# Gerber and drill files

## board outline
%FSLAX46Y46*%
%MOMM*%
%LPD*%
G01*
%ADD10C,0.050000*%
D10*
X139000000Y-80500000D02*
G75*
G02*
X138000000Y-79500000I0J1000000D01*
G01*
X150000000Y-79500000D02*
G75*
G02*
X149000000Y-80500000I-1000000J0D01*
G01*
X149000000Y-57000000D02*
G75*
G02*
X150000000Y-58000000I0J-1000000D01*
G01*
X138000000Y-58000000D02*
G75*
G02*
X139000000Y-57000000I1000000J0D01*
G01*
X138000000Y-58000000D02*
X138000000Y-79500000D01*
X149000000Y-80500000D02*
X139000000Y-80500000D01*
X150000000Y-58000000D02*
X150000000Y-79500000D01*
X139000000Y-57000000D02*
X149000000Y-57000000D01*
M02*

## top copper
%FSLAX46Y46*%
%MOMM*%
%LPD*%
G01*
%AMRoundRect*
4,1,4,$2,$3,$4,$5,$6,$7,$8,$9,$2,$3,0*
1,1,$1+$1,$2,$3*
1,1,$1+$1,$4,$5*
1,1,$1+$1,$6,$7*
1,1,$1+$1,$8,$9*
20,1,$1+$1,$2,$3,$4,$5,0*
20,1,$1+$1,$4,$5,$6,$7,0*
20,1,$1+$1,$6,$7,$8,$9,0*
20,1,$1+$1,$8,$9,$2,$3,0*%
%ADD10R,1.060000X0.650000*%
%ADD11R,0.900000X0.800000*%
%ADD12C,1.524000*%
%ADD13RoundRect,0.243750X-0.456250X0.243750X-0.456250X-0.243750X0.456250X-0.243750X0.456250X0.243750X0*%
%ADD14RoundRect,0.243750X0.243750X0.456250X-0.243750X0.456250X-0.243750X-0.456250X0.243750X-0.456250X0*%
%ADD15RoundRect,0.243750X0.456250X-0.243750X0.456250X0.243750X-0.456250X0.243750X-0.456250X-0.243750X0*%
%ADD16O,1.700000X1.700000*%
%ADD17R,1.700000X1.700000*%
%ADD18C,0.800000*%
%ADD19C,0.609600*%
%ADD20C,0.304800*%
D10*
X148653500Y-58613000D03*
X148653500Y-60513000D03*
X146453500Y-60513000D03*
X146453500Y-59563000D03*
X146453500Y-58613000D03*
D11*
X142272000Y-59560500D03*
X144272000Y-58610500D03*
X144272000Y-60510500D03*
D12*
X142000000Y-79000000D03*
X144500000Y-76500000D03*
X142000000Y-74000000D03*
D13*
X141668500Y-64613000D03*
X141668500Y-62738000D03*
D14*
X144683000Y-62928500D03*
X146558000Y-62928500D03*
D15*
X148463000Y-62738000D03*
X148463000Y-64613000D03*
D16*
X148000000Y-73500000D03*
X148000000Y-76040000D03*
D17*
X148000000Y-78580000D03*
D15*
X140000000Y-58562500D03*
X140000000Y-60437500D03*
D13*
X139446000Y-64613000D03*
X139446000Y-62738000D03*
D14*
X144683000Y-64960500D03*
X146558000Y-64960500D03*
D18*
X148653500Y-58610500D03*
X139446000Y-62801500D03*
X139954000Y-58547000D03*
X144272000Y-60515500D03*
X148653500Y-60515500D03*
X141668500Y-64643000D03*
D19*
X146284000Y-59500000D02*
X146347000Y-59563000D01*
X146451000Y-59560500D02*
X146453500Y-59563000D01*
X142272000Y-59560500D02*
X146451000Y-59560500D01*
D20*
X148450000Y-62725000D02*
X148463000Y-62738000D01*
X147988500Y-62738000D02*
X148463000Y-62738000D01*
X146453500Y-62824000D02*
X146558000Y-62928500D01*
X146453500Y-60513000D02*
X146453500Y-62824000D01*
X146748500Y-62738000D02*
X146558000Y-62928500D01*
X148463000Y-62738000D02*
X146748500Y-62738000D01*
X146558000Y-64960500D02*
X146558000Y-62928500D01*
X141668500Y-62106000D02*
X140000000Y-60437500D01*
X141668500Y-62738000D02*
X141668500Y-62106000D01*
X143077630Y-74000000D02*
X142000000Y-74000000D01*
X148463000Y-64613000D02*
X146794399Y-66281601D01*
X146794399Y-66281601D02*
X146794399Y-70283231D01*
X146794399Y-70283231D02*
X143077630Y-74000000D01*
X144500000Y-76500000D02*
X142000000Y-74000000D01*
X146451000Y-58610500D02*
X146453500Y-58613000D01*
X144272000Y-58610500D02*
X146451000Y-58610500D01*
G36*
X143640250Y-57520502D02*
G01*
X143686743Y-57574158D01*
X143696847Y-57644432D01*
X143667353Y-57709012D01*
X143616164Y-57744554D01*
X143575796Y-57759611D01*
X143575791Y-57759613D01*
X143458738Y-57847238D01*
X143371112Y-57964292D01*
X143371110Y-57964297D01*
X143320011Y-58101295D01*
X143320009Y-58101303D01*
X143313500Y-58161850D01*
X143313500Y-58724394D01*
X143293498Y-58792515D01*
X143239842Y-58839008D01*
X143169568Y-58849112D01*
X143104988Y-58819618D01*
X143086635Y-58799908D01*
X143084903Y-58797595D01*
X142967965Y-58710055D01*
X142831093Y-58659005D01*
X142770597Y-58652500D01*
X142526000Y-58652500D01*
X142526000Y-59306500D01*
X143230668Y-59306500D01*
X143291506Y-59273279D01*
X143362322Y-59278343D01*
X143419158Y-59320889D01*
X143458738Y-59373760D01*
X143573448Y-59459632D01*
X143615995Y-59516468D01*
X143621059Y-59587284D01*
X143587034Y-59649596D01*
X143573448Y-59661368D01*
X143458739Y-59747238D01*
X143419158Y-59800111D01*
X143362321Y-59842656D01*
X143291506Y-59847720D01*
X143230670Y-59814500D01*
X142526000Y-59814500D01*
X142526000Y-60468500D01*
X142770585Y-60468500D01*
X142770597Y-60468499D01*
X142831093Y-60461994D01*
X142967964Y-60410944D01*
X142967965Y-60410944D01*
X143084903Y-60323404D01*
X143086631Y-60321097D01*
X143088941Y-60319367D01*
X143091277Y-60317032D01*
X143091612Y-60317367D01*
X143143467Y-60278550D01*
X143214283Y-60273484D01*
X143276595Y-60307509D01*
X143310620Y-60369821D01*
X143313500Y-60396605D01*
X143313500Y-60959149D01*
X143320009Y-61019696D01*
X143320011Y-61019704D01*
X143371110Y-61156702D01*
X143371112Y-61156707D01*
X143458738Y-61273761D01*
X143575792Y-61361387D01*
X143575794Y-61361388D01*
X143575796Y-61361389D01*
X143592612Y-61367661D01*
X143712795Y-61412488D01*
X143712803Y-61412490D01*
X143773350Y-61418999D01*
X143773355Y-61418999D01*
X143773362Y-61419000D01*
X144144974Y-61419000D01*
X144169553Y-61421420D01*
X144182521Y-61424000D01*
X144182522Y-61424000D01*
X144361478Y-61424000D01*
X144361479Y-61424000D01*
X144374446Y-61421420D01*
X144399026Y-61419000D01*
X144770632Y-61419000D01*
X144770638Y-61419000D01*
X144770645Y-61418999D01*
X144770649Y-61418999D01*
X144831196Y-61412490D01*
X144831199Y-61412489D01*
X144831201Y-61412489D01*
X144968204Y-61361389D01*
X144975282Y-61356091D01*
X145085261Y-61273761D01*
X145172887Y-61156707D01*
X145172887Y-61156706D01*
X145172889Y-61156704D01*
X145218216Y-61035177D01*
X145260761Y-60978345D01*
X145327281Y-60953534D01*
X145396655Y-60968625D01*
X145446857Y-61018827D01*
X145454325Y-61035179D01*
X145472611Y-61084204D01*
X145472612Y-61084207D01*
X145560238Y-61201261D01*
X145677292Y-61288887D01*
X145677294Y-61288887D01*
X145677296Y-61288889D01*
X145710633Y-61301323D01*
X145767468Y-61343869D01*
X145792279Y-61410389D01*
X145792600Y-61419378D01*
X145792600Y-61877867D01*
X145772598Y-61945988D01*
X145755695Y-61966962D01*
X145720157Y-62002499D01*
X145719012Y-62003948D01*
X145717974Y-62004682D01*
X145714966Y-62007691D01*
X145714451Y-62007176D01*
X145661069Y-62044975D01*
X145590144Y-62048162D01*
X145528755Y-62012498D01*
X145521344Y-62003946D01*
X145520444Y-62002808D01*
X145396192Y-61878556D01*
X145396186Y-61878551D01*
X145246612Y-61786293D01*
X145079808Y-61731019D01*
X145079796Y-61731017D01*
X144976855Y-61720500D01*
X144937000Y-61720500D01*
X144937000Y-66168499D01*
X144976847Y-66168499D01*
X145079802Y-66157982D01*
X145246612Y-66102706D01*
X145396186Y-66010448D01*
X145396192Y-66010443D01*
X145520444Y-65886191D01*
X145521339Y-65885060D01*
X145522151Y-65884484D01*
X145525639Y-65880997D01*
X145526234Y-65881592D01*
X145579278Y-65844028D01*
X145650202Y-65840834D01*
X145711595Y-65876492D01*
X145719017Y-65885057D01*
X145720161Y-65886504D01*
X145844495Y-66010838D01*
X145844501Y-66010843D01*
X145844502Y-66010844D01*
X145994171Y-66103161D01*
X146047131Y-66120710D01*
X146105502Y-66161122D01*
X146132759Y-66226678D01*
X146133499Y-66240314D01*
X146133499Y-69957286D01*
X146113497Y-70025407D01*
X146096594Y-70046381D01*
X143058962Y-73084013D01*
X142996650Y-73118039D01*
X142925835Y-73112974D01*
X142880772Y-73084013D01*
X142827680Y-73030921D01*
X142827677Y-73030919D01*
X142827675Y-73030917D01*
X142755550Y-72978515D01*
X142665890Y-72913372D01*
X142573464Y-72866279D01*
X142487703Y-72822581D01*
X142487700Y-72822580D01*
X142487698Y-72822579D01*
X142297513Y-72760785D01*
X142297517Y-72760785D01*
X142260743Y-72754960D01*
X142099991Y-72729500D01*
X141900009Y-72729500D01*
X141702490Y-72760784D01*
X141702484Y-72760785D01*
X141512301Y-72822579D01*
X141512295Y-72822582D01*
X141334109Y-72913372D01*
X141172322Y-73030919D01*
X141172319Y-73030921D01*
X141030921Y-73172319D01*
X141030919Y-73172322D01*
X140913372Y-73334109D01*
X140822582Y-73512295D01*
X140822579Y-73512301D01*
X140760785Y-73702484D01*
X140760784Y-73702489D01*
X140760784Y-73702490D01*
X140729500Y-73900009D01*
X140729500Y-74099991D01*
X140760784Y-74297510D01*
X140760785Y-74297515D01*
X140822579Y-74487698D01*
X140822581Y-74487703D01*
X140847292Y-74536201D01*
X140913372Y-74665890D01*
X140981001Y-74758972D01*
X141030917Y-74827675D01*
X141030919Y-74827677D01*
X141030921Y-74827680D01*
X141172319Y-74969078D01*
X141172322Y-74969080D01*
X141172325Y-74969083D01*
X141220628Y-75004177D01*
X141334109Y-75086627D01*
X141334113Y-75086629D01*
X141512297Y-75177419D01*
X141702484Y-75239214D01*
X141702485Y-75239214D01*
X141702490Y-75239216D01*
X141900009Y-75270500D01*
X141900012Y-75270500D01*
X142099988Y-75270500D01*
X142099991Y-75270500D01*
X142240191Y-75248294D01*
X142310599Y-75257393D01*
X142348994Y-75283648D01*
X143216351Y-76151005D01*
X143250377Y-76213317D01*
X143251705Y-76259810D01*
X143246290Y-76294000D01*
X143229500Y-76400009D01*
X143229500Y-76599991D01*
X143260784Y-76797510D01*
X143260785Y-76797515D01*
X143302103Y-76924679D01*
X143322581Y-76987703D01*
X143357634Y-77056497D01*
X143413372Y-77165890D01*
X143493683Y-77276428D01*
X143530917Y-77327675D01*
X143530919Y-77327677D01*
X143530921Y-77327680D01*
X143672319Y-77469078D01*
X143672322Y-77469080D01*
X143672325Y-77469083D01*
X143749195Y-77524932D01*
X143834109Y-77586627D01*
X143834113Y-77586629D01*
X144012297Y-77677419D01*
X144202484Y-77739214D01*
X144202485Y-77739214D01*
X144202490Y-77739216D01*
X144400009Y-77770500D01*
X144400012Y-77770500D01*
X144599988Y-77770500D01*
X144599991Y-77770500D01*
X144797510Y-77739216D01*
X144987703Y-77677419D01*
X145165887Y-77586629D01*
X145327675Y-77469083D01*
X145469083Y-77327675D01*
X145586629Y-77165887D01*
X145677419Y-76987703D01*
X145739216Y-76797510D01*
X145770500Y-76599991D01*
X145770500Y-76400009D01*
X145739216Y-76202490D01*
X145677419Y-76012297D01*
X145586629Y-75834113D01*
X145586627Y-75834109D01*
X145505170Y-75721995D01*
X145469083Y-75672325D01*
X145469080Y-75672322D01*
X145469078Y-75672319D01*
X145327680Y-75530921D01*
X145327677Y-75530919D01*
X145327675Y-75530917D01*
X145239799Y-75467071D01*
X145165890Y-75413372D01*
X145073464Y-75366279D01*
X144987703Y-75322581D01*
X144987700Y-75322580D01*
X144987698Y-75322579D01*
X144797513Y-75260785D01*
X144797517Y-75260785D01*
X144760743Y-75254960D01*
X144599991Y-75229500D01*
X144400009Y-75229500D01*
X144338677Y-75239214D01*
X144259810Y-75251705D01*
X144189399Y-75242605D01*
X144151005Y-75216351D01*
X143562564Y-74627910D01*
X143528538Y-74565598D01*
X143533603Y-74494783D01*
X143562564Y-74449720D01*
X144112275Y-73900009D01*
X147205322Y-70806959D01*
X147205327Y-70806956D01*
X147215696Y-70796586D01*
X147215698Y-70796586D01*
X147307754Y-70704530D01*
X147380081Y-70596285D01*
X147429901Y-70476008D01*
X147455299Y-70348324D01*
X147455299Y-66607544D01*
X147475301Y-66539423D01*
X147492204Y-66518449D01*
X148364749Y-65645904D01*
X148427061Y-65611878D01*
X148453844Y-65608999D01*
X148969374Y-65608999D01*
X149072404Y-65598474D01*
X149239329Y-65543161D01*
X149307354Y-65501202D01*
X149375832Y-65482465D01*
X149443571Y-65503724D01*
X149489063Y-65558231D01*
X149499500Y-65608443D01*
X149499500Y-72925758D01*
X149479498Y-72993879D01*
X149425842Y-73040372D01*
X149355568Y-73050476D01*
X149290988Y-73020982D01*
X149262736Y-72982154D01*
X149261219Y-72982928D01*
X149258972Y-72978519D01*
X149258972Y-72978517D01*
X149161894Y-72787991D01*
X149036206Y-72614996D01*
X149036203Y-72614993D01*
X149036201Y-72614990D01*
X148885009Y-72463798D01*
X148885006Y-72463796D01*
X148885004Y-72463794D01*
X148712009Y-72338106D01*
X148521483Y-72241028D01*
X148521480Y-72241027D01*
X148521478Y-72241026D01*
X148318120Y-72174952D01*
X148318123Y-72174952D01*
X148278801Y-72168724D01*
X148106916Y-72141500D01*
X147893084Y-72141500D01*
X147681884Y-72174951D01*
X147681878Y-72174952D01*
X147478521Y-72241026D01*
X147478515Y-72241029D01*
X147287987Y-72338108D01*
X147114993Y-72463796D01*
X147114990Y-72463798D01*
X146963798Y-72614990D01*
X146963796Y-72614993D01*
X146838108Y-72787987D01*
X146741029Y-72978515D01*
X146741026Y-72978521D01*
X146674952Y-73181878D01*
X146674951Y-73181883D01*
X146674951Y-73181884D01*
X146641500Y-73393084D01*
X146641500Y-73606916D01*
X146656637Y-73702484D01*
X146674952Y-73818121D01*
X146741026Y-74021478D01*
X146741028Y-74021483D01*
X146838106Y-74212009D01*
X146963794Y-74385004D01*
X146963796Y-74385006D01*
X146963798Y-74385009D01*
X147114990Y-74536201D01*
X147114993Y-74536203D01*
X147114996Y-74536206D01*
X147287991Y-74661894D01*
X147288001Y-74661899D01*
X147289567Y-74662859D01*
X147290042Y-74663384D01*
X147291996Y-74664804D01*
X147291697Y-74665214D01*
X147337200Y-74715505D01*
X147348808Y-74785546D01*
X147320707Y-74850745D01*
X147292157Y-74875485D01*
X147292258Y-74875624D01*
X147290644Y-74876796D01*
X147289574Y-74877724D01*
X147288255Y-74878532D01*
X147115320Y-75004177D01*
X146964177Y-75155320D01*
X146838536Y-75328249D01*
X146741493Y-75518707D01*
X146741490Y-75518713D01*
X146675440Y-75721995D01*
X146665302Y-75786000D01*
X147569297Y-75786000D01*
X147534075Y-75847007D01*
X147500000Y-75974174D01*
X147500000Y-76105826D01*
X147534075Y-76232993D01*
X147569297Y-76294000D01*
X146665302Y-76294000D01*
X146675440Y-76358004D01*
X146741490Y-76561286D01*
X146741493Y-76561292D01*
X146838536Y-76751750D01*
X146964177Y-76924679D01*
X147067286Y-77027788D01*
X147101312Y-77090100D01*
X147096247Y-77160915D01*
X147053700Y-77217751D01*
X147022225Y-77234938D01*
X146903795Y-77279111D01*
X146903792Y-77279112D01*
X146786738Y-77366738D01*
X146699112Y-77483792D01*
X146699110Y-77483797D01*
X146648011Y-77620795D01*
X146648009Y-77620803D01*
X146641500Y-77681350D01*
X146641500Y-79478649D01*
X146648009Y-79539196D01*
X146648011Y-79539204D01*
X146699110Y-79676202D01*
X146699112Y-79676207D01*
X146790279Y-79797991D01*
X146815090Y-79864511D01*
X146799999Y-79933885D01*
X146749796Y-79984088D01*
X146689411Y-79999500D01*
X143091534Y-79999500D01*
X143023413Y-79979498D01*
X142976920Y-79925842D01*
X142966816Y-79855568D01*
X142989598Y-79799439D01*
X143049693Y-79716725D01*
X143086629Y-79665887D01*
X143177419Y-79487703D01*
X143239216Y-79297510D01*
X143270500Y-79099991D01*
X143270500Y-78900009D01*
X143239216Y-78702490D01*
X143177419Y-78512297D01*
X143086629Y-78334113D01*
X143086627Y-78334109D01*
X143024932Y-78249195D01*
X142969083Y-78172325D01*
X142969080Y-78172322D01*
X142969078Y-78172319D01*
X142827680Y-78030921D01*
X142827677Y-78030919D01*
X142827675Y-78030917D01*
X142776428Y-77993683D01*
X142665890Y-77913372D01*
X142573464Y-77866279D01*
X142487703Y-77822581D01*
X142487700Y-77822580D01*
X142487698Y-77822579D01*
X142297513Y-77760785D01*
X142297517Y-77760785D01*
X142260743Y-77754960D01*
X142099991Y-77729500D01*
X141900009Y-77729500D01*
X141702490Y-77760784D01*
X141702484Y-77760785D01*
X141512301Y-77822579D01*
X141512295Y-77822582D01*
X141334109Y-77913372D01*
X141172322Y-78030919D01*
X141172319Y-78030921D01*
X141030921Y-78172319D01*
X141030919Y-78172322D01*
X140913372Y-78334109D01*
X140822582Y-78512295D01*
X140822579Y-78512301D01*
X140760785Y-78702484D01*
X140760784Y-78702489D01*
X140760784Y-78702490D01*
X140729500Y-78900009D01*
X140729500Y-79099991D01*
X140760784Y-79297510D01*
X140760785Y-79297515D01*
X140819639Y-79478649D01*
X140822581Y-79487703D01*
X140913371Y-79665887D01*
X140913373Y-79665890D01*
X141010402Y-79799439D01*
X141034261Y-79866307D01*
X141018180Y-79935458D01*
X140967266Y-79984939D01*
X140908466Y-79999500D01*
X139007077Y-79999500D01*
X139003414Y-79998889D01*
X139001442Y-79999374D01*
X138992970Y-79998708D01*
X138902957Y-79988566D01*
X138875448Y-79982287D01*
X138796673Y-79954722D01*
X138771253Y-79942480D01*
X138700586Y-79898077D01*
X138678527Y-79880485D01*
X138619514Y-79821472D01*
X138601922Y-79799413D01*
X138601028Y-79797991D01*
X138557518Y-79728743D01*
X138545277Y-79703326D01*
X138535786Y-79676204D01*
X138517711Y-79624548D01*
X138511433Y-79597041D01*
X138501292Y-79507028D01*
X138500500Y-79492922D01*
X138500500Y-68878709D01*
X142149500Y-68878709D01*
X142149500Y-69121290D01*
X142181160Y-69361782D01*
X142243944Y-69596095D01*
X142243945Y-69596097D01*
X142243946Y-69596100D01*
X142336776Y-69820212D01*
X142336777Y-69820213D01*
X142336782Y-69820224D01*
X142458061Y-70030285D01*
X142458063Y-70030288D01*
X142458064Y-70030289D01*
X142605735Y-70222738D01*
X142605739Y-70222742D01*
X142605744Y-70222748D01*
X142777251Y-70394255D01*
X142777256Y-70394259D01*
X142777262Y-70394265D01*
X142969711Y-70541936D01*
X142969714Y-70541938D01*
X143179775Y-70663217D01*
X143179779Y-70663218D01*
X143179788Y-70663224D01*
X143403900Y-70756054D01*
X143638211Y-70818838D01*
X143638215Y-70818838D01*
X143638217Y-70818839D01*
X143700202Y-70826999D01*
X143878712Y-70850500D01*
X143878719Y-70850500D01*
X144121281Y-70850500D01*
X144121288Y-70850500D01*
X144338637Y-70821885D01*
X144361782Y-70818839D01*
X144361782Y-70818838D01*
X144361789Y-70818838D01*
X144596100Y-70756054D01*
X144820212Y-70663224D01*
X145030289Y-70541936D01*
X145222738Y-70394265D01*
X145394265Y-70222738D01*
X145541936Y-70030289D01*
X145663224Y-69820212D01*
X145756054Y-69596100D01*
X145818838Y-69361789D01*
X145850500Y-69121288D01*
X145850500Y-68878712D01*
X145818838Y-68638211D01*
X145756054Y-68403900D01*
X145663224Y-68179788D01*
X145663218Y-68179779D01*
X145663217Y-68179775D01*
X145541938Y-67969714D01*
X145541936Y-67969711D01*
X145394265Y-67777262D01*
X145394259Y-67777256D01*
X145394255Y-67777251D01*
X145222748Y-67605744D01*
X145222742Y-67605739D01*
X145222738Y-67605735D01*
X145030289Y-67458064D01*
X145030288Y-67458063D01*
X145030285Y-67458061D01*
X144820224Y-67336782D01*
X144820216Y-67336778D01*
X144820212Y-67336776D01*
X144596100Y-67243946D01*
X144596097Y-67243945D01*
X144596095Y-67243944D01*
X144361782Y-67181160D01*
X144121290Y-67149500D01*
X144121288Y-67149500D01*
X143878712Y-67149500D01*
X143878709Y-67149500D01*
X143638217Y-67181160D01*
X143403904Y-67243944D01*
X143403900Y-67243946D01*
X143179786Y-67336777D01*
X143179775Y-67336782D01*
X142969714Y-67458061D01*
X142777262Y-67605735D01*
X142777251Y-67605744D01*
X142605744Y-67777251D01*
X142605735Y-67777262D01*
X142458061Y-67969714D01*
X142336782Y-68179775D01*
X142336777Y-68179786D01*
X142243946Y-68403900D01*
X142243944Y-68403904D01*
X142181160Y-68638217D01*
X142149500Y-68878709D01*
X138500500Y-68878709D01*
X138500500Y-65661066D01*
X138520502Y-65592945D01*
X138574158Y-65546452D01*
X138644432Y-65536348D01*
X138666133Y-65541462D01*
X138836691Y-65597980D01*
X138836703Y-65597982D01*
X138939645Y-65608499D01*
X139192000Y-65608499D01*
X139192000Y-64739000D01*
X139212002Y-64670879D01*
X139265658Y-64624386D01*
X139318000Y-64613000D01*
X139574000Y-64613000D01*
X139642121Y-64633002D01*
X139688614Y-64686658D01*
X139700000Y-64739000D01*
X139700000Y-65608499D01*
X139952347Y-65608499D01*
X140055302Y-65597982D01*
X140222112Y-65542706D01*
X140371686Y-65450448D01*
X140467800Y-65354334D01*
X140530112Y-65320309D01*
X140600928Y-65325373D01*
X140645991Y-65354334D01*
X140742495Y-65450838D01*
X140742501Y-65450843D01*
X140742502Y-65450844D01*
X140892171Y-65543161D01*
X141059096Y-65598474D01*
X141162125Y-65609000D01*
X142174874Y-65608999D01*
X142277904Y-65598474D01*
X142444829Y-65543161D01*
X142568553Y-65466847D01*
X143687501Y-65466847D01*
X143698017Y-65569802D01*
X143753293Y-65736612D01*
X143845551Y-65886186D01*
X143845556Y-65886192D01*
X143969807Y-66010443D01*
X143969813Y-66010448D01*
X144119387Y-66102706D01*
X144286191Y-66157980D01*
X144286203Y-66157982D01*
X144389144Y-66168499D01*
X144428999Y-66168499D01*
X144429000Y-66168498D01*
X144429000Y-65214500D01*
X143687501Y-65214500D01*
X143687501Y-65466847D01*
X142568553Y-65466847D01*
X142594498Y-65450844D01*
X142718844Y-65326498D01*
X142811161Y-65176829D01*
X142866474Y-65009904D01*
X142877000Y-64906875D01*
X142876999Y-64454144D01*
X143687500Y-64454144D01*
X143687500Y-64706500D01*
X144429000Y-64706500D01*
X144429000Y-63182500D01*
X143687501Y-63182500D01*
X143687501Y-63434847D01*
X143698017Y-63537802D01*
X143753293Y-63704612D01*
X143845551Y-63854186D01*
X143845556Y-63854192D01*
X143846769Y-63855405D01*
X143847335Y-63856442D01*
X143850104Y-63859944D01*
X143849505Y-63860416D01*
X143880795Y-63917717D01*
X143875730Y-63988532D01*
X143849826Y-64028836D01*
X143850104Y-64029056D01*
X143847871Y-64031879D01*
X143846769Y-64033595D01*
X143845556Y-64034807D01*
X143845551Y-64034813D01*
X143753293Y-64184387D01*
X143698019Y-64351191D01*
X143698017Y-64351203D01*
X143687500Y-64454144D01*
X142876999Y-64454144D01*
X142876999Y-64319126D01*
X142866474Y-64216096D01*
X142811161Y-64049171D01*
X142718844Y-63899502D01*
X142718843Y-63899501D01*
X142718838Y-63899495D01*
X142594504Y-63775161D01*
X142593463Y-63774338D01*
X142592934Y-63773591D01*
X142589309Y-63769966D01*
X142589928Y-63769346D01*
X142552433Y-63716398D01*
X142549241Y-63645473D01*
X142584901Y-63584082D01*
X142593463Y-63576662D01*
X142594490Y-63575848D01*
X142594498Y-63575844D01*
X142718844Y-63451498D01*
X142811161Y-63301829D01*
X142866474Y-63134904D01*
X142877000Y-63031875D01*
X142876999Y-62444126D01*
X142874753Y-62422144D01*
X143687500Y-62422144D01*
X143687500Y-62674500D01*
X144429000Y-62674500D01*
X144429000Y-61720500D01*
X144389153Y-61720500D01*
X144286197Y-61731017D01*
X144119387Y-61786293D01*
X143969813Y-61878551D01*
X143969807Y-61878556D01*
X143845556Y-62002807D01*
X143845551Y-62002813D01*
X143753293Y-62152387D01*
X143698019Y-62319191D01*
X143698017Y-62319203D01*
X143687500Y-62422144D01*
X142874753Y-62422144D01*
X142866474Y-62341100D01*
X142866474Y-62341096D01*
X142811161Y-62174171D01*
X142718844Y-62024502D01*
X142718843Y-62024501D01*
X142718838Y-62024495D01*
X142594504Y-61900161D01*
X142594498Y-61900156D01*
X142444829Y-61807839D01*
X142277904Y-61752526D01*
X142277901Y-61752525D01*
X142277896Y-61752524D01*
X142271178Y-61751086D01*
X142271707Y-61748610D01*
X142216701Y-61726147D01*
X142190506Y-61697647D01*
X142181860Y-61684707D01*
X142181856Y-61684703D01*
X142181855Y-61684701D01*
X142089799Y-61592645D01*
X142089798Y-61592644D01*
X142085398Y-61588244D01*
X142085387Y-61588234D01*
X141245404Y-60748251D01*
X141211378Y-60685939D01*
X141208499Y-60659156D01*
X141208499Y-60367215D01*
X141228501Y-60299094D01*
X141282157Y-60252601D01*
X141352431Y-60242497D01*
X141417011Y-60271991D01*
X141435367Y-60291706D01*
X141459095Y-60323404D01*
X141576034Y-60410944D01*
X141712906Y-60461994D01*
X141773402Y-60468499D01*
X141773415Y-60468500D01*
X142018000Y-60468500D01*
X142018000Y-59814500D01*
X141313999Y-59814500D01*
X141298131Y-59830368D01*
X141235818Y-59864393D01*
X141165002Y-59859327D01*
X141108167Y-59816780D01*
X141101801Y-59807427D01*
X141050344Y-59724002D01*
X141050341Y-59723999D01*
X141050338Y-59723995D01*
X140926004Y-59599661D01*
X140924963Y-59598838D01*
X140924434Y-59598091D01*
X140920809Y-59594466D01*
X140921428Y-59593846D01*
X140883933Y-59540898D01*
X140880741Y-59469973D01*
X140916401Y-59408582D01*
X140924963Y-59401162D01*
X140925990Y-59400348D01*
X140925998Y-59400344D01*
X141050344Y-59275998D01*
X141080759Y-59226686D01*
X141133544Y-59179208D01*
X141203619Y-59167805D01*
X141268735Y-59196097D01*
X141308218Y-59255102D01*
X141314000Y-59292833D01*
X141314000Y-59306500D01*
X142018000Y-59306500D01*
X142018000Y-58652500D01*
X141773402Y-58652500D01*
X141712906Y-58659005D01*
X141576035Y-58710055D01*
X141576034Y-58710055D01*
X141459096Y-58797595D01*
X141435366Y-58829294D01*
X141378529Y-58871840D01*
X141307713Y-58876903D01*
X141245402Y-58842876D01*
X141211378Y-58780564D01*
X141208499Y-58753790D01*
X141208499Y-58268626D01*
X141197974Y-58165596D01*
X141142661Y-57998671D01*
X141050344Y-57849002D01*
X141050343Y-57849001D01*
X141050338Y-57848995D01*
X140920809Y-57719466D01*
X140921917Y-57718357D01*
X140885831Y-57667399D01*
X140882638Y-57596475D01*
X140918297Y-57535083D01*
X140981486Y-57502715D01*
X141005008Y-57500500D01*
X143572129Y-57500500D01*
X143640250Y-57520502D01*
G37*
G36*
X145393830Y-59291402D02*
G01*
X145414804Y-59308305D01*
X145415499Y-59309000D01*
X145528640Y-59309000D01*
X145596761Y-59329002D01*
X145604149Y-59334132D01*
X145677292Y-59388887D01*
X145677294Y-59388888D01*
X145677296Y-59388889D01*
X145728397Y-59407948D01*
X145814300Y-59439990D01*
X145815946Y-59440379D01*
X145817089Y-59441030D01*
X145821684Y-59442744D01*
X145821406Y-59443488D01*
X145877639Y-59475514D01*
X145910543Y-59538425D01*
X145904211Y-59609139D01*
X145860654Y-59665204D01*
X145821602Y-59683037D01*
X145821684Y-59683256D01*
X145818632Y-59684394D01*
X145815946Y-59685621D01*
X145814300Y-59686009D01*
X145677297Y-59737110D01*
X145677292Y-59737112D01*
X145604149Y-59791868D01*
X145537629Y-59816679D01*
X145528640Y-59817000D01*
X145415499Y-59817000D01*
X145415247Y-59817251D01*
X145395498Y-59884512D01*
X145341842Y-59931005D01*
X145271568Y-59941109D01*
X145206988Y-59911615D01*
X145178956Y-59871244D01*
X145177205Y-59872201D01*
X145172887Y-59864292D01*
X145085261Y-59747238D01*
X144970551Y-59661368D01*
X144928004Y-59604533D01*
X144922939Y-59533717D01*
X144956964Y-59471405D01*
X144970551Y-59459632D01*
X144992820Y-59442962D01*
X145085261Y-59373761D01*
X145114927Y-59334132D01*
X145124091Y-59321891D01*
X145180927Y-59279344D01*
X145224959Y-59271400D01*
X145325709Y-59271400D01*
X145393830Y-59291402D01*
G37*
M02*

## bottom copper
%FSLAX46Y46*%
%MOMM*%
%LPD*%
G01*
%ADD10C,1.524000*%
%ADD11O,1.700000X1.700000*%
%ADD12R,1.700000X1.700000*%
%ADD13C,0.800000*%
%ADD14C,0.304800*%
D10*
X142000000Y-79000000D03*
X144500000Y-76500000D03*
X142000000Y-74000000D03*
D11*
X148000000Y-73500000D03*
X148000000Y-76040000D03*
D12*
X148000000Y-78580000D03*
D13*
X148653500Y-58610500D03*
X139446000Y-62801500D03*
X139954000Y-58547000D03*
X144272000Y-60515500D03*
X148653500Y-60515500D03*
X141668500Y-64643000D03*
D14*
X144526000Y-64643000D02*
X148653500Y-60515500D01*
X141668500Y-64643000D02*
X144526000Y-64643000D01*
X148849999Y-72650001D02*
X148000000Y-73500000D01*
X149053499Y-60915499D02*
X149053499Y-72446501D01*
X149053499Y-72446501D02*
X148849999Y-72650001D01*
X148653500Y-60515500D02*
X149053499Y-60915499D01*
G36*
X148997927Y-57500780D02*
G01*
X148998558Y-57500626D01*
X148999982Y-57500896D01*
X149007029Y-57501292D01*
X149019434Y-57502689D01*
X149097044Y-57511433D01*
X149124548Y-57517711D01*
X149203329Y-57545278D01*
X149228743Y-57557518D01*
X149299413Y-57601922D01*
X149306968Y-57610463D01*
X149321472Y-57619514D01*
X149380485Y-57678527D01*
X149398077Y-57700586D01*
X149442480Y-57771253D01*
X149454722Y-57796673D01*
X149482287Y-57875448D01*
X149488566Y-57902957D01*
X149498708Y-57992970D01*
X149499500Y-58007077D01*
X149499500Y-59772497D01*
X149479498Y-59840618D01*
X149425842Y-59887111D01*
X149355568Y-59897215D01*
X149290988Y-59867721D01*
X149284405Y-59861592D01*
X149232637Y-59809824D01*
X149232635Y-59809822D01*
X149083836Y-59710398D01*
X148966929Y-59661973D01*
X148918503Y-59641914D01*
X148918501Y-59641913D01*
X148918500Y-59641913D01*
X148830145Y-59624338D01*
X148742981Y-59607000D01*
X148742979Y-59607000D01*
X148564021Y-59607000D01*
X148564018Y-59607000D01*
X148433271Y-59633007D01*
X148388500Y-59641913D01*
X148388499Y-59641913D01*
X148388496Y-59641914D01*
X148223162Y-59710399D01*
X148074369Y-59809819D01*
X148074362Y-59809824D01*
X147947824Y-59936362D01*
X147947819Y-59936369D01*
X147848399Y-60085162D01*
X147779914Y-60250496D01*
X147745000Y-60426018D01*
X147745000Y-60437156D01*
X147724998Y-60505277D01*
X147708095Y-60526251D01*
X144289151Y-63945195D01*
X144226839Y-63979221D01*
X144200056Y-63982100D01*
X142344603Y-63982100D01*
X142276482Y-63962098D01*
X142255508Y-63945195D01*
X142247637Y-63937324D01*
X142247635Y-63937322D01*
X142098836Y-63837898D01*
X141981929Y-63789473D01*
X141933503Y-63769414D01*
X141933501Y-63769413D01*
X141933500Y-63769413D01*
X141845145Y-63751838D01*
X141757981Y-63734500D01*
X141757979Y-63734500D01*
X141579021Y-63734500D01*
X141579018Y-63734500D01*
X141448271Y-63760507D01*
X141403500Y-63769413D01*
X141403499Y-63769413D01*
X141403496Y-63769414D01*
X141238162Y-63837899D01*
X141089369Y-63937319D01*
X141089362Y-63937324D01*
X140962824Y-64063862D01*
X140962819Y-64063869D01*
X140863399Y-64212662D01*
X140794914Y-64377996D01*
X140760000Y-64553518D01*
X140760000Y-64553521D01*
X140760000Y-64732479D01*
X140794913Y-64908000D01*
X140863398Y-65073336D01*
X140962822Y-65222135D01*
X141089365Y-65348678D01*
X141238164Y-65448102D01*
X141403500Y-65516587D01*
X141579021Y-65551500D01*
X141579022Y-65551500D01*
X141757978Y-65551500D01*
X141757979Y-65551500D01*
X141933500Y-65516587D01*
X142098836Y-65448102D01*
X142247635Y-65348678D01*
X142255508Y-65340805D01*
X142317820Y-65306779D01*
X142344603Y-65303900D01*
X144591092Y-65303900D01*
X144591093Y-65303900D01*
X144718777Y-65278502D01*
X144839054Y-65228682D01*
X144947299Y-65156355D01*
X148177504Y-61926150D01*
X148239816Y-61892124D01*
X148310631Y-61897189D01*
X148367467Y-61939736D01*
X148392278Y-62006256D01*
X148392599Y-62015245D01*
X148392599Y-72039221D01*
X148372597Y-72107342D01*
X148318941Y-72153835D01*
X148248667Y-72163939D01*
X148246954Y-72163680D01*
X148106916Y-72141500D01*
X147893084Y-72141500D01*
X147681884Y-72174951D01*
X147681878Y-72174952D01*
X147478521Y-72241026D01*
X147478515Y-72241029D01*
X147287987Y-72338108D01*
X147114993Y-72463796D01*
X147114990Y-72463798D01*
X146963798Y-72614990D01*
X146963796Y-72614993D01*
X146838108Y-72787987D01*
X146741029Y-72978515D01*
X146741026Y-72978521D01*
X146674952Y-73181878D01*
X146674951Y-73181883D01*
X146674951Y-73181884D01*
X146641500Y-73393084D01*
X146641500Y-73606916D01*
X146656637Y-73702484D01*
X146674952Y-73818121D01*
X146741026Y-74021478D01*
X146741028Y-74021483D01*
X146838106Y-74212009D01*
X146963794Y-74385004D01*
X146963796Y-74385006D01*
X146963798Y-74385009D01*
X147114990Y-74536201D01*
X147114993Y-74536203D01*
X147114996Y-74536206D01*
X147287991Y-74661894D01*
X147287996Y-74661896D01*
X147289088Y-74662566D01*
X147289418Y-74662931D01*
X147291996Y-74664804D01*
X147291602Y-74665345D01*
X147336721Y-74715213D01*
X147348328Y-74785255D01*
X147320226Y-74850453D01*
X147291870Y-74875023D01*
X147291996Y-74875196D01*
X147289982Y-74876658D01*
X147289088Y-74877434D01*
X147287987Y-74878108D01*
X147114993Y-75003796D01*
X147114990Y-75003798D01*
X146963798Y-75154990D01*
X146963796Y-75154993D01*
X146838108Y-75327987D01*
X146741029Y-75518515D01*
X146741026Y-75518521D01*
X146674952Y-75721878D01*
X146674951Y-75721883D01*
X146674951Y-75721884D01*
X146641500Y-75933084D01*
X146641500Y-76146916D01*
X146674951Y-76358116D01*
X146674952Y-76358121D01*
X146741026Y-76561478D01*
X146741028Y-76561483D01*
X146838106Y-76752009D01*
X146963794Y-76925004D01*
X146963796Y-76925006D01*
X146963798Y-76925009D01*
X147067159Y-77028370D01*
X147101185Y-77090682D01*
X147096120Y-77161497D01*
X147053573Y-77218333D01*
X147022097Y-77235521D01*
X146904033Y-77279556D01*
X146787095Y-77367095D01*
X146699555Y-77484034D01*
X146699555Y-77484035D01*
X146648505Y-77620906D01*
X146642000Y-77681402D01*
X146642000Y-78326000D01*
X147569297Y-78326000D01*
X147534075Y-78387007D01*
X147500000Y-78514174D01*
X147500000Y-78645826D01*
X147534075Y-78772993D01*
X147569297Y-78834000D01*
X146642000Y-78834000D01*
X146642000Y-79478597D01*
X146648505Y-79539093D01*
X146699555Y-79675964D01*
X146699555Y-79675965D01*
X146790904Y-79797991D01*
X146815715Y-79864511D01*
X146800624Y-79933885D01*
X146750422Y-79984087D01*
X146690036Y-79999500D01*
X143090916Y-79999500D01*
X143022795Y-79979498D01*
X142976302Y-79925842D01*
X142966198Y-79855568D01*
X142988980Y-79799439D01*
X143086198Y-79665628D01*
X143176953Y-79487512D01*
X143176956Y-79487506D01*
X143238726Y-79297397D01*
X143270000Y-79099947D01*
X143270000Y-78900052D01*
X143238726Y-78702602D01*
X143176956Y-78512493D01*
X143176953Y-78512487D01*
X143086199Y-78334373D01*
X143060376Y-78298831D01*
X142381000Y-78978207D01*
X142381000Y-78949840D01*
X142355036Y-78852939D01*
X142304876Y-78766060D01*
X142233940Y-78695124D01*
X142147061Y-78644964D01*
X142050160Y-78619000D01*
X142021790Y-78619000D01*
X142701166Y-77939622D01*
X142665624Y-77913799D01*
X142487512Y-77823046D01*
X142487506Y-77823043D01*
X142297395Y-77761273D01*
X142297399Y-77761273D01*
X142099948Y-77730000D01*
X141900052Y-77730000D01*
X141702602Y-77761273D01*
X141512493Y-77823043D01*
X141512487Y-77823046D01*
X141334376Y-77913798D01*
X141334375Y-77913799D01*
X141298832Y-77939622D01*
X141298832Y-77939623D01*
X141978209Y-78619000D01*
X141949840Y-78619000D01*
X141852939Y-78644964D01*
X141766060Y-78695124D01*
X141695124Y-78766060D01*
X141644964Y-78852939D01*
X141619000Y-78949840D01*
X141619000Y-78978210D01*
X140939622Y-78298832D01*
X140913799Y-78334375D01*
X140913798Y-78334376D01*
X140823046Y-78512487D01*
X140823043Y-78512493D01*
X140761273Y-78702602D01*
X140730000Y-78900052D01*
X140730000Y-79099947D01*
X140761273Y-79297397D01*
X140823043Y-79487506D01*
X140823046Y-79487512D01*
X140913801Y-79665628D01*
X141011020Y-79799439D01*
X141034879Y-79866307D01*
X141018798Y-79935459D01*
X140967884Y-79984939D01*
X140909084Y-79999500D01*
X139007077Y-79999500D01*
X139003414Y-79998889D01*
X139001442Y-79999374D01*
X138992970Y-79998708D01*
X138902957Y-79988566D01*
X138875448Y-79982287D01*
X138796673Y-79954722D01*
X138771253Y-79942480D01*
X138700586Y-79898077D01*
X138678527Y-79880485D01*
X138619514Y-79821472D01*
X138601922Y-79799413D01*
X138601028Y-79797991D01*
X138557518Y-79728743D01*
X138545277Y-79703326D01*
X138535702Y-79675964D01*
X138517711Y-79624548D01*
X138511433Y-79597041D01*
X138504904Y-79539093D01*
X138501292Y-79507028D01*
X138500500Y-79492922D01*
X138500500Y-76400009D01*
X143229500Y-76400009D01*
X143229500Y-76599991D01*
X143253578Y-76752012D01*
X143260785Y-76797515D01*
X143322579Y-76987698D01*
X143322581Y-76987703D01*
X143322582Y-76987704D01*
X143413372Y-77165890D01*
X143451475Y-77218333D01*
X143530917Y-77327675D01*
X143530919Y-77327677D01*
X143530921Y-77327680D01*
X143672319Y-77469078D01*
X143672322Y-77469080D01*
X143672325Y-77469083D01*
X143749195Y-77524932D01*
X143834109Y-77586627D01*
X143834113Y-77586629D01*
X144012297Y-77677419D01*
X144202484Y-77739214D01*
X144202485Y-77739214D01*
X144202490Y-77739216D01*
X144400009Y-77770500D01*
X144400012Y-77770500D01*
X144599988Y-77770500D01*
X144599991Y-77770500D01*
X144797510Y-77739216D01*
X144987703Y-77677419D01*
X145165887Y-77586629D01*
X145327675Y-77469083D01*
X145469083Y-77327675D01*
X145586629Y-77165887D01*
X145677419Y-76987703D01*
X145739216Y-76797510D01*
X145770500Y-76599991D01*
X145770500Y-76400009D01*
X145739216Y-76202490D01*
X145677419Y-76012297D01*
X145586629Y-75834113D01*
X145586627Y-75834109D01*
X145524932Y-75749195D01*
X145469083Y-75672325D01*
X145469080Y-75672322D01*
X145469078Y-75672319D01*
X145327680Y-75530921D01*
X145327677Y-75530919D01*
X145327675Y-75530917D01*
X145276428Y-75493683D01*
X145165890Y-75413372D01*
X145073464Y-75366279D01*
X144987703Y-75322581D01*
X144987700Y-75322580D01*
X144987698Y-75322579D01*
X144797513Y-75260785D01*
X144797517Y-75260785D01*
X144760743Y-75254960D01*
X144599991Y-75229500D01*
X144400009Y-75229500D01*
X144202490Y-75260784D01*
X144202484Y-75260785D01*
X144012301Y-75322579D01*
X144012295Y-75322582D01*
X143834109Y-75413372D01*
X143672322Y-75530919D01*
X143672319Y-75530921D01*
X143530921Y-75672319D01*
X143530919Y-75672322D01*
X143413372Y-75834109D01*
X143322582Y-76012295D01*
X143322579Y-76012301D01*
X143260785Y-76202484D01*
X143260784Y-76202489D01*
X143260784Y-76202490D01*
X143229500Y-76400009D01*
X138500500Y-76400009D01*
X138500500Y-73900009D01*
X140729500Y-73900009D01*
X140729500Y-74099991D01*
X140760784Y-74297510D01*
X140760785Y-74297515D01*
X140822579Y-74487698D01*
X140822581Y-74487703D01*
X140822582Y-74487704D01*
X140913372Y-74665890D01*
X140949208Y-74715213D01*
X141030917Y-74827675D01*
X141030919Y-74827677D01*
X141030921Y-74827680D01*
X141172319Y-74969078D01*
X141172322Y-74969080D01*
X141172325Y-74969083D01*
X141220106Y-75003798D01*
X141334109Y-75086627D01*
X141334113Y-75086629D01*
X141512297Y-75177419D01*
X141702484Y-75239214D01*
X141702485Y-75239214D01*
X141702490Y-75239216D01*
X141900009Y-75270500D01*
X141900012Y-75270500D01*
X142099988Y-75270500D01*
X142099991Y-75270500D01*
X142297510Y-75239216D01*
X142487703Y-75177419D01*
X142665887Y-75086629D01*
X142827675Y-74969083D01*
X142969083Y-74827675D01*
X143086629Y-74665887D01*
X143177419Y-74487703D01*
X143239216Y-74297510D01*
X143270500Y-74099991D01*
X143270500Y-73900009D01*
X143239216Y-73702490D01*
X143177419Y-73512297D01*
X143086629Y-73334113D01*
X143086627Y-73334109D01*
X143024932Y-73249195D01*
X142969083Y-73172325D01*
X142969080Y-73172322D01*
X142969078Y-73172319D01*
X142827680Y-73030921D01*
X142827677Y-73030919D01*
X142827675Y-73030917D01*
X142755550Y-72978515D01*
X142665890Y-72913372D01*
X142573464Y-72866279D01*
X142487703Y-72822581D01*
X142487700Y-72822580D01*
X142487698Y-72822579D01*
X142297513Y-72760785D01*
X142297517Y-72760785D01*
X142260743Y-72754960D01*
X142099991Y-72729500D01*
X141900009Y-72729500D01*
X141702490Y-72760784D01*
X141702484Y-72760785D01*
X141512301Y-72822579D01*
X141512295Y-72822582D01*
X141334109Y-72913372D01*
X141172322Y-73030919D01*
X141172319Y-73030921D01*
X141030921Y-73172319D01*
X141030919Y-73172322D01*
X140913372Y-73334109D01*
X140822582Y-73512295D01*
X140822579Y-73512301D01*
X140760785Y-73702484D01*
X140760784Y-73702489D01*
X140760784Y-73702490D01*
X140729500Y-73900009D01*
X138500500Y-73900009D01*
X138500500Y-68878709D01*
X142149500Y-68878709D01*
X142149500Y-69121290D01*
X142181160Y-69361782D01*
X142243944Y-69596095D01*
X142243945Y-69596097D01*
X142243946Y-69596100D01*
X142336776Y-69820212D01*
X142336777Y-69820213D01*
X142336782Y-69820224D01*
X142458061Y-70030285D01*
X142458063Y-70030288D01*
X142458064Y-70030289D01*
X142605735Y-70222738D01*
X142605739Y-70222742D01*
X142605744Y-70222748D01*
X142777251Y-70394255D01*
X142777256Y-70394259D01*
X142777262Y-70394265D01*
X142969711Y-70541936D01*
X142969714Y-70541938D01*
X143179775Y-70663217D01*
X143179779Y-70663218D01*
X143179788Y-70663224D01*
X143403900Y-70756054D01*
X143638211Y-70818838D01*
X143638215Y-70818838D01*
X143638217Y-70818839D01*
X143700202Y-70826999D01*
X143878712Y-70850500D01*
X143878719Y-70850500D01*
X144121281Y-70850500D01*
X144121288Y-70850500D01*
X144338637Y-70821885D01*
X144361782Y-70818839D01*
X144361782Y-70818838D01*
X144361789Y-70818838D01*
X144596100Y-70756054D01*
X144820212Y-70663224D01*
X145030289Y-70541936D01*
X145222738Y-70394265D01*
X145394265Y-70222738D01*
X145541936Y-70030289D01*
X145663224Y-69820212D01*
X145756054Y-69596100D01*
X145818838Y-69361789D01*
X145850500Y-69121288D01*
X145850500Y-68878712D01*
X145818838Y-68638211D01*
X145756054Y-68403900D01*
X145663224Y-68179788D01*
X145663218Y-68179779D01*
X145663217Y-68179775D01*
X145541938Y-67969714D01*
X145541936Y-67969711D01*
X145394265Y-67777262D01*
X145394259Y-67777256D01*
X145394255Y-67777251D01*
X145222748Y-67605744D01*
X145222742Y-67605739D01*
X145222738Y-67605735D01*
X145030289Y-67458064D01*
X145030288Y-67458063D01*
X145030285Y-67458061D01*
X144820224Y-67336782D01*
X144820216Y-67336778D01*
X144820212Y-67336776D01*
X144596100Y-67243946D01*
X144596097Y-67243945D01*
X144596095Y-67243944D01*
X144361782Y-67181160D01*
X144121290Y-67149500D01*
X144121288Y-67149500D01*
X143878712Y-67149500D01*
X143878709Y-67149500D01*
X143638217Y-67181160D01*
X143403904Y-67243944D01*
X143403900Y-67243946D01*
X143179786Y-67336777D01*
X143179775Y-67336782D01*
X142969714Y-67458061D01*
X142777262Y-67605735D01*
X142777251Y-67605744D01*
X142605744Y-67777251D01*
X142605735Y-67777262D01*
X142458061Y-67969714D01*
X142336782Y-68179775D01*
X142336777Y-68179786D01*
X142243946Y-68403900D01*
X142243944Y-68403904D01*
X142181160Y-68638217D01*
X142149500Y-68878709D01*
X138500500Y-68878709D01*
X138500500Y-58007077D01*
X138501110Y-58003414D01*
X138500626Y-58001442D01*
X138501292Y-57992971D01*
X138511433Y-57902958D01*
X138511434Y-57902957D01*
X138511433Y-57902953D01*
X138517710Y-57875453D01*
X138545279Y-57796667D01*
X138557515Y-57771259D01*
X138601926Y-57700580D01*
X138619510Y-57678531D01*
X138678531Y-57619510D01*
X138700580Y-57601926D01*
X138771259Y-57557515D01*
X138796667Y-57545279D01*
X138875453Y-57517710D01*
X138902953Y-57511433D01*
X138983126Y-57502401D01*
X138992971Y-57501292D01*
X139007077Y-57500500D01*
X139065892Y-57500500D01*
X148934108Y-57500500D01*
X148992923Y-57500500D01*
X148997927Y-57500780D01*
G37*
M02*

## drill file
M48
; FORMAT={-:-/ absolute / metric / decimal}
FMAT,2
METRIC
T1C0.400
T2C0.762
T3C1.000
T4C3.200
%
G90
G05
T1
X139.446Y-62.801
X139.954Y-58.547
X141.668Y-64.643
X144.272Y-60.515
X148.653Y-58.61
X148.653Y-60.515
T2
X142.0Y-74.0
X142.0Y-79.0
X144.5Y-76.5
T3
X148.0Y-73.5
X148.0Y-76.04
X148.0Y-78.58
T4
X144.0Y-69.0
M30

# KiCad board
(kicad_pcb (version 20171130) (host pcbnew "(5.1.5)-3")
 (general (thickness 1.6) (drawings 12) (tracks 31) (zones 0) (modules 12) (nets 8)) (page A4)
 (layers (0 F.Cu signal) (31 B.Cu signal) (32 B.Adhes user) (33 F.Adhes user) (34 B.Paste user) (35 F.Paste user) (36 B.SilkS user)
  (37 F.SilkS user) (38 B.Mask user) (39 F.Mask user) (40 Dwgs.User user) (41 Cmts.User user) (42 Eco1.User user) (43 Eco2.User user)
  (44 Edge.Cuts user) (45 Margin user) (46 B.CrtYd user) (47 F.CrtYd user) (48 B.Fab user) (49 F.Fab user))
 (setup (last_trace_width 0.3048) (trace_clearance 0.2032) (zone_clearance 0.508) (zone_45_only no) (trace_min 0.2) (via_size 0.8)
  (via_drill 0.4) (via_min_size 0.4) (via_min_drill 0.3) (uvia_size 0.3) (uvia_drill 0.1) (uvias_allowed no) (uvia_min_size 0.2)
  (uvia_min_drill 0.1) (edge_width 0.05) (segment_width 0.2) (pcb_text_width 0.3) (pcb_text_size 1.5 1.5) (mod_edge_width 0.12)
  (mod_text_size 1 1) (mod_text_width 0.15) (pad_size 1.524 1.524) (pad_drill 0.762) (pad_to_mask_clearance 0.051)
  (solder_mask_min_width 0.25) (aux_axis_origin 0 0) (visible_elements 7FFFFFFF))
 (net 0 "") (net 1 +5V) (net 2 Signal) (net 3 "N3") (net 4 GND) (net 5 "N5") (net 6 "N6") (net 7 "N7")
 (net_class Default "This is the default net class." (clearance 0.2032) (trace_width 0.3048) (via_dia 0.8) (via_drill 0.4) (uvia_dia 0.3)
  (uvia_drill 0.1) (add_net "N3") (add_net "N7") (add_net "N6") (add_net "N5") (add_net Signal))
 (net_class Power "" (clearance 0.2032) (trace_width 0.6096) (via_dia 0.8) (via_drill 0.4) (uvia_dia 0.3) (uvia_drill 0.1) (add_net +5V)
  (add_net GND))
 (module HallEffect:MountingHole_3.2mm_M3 (layer F.Cu) (at 144 69)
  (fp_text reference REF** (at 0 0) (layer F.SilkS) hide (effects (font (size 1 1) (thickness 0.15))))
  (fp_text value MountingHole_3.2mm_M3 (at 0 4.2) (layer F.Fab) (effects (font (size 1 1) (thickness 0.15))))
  (pad 1 np_thru_hole circle (at 0 0) (size 3.2 3.2) (drill 3.2) (layers *.Cu *.Mask)))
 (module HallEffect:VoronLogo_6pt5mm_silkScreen (layer B.Cu) (at 144 61 270)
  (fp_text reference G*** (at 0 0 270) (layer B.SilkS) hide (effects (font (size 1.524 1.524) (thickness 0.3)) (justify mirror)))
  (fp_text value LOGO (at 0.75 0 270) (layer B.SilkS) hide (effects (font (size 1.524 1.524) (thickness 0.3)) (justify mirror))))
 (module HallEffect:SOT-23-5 (layer F.Cu) (at 147.5535 59.563)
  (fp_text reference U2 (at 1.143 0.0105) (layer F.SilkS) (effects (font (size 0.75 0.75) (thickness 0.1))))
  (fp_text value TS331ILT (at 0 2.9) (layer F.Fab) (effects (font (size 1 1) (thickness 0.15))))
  (pad 5 smd rect (at 1.1 -0.95) (size 1.06 0.65) (layers F.Cu F.Paste F.Mask) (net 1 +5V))
  (pad 4 smd rect (at 1.1 0.95) (size 1.06 0.65) (layers F.Cu F.Paste F.Mask) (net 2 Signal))
  (pad 3 smd rect (at -1.1 0.95) (size 1.06 0.65) (layers F.Cu F.Paste F.Mask) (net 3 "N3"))
  (pad 2 smd rect (at -1.1 0) (size 1.06 0.65) (layers F.Cu F.Paste F.Mask) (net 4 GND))
  (pad 1 smd rect (at -1.1 -0.95) (size 1.06 0.65) (layers F.Cu F.Paste F.Mask) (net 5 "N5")))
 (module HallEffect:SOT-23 (layer F.Cu) (at 143.272 59.5605 180)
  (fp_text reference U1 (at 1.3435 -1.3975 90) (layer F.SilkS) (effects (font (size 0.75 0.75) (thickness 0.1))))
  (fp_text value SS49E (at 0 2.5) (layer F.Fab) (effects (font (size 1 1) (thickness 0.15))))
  (pad 3 smd rect (at 1 0 180) (size 0.9 0.8) (layers F.Cu F.Paste F.Mask) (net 4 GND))
  (pad 2 smd rect (at -1 0.95 180) (size 0.9 0.8) (layers F.Cu F.Paste F.Mask) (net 5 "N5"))
  (pad 1 smd rect (at -1 -0.95 180) (size 0.9 0.8) (layers F.Cu F.Paste F.Mask) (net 1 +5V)))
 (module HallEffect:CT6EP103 (layer F.Cu) (at 142 76.5 270)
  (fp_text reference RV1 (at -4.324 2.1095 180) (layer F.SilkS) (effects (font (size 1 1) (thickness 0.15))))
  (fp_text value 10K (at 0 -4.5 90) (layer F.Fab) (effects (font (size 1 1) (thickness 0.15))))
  (pad 3 thru_hole circle (at 2.5 0 270) (size 1.524 1.524) (drill 0.762) (layers *.Cu *.Mask) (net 1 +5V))
  (pad 2 thru_hole circle (at 0 -2.5 270) (size 1.524 1.524) (drill 0.762) (layers *.Cu *.Mask) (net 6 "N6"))
  (pad 1 thru_hole circle (at -2.5 0 270) (size 1.524 1.524) (drill 0.762) (layers *.Cu *.Mask) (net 6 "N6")))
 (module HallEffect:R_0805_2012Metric (layer F.Cu) (at 141.6685 63.6755 270)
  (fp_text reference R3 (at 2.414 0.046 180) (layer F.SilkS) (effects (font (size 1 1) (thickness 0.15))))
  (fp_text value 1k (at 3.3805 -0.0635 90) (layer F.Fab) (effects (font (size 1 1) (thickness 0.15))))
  (pad 2 smd roundrect (at 0.9375 0 270) (size 0.975 1.4) (layers F.Cu F.Paste F.Mask) (roundrect_rratio 0.25) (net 2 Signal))
  (pad 1 smd roundrect (at -0.9375 0 270) (size 0.975 1.4) (layers F.Cu F.Paste F.Mask) (roundrect_rratio 0.25) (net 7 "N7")))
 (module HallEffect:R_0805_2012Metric (layer F.Cu) (at 145.6205 62.9285 180)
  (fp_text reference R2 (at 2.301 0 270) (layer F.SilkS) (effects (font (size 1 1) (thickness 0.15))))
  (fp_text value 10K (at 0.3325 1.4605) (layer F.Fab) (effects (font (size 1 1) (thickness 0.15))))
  (pad 2 smd roundrect (at 0.9375 0 180) (size 0.975 1.4) (layers F.Cu F.Paste F.Mask) (roundrect_rratio 0.25) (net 4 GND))
  (pad 1 smd roundrect (at -0.9375 0 180) (size 0.975 1.4) (layers F.Cu F.Paste F.Mask) (roundrect_rratio 0.25) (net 3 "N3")))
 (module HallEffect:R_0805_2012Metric (layer F.Cu) (at 148.463 63.6755 90)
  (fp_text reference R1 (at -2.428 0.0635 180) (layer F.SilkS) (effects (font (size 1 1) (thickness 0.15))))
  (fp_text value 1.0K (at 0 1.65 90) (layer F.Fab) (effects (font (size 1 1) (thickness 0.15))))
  (pad 2 smd roundrect (at 0.9375 0 90) (size 0.975 1.4) (layers F.Cu F.Paste F.Mask) (roundrect_rratio 0.25) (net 3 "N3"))
  (pad 1 smd roundrect (at -0.9375 0 90) (size 0.975 1.4) (layers F.Cu F.Paste F.Mask) (roundrect_rratio 0.25) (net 6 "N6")))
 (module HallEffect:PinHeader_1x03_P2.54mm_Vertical (layer F.Cu) (at 148 78.58 180)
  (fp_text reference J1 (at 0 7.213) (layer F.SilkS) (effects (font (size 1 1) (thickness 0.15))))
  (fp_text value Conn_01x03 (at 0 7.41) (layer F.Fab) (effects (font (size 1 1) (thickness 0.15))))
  (pad 3 thru_hole oval (at 0 5.08 180) (size 1.7 1.7) (drill 1) (layers *.Cu *.Mask) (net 2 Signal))
  (pad 2 thru_hole oval (at 0 2.54 180) (size 1.7 1.7) (drill 1) (layers *.Cu *.Mask) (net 4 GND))
  (pad 1 thru_hole rect (at 0 0 180) (size 1.7 1.7) (drill 1) (layers *.Cu *.Mask) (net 1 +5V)))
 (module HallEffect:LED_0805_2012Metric (layer F.Cu) (at 140 59.5 90)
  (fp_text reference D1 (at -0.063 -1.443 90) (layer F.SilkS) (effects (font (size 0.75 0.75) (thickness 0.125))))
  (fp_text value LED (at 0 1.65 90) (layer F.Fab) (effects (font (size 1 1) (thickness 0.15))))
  (pad 2 smd roundrect (at 0.9375 0 90) (size 0.975 1.4) (layers F.Cu F.Paste F.Mask) (roundrect_rratio 0.25) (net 1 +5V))
  (pad 1 smd roundrect (at -0.9375 0 90) (size 0.975 1.4) (layers F.Cu F.Paste F.Mask) (roundrect_rratio 0.25) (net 7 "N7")))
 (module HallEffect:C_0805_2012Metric (layer F.Cu) (at 139.446 63.6755 270)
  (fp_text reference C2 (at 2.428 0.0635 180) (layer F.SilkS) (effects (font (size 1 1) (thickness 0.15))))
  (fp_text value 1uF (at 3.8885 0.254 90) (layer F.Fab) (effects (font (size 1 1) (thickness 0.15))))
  (pad 2 smd roundrect (at 0.9375 0 270) (size 0.975 1.4) (layers F.Cu F.Paste F.Mask) (roundrect_rratio 0.25) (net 4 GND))
  (pad 1 smd roundrect (at -0.9375 0 270) (size 0.975 1.4) (layers F.Cu F.Paste F.Mask) (roundrect_rratio 0.25) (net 1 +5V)))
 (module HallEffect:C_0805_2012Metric (layer F.Cu) (at 145.6205 64.9605 180)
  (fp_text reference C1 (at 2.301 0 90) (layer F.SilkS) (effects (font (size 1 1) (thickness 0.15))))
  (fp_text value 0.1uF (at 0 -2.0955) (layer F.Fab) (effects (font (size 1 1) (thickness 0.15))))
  (pad 2 smd roundrect (at 0.9375 0 180) (size 0.975 1.4) (layers F.Cu F.Paste F.Mask) (roundrect_rratio 0.25) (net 4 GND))
  (pad 1 smd roundrect (at -0.9375 0 180) (size 0.975 1.4) (layers F.Cu F.Paste F.Mask) (roundrect_rratio 0.25) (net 3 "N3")))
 (gr_arc (start 139 79.5) (end 138 79.5) (angle -90) (layer Edge.Cuts) (width 0.05))
 (gr_arc (start 149 79.5) (end 149 80.5) (angle -90) (layer Edge.Cuts) (width 0.05))
 (gr_arc (start 149 58) (end 150 58) (angle -90) (layer Edge.Cuts) (width 0.05))
 (gr_arc (start 139 58) (end 139 57) (angle -90) (layer Edge.Cuts) (width 0.05))
 (gr_line (start 138 58) (end 138 79.5) (layer Edge.Cuts) (width 0.05))
 (gr_line (start 149 80.5) (end 139 80.5) (layer Edge.Cuts) (width 0.05))
 (gr_line (start 150 58) (end 150 79.5) (layer Edge.Cuts) (width 0.05))
 (gr_line (start 139 57) (end 149 57) (layer Edge.Cuts) (width 0.05))
 (segment (start 146.284 59.5) (end 146.347 59.563) (width 0.6096) (layer F.Cu) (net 4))
 (segment (start 146.451 59.5605) (end 146.4535 59.563) (width 0.6096) (layer F.Cu) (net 4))
 (segment (start 142.272 59.5605) (end 146.451 59.5605) (width 0.6096) (layer F.Cu) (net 4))
 (segment (start 148.45 62.725) (end 148.463 62.738) (width 0.3048) (layer F.Cu) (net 3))
 (segment (start 147.9885 62.738) (end 148.463 62.738) (width 0.3048) (layer F.Cu) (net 3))
 (segment (start 146.4535 62.824) (end 146.558 62.9285) (width 0.3048) (layer F.Cu) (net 3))
 (segment (start 146.4535 60.513) (end 146.4535 62.824) (width 0.3048) (layer F.Cu) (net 3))
 (segment (start 146.7485 62.738) (end 146.558 62.9285) (width 0.3048) (layer F.Cu) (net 3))
 (segment (start 148.463 62.738) (end 146.7485 62.738) (width 0.3048) (layer F.Cu) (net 3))
 (segment (start 146.558 64.9605) (end 146.558 62.9285) (width 0.3048) (layer F.Cu) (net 3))
 (via (at 148.6535 58.6105) (size 0.8) (drill 0.4) (layers F.Cu B.Cu) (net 1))
 (via (at 139.446 62.8015) (size 0.8) (drill 0.4) (layers F.Cu B.Cu) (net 1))
 (via (at 139.954 58.547) (size 0.8) (drill 0.4) (layers F.Cu B.Cu) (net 1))
 (via (at 144.272 60.5155) (size 0.8) (drill 0.4) (layers F.Cu B.Cu) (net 1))
 (segment (start 141.6685 62.106) (end 140 60.4375) (width 0.3048) (layer F.Cu) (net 7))
 (segment (start 141.6685 62.738) (end 141.6685 62.106) (width 0.3048) (layer F.Cu) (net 7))
 (via (at 148.6535 60.5155) (size 0.8) (drill 0.4) (layers F.Cu B.Cu) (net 2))
 (via (at 141.6685 64.643) (size 0.8) (drill 0.4) (layers F.Cu B.Cu) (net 2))
 (segment (start 144.526 64.643) (end 148.6535 60.5155) (width 0.3048) (layer B.Cu) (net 2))
 (segment (start 141.6685 64.643) (end 144.526 64.643) (width 0.3048) (layer B.Cu) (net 2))
 (segment (start 148.849999 72.650001) (end 148 73.5) (width 0.3048) (layer B.Cu) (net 2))
 (segment (start 149.053499 60.915499) (end 149.053499 72.446501) (width 0.3048) (layer B.Cu) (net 2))
 (segment (start 149.053499 72.446501) (end 148.849999 72.650001) (width 0.3048) (layer B.Cu) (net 2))
 (segment (start 148.6535 60.5155) (end 149.053499 60.915499) (width 0.3048) (layer B.Cu) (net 2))
 (segment (start 143.07763 74) (end 142 74) (width 0.3048) (layer F.Cu) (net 6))
 (segment (start 148.463 64.613) (end 146.794399 66.281601) (width 0.3048) (layer F.Cu) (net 6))
 (segment (start 146.794399 66.281601) (end 146.794399 70.283231) (width 0.3048) (layer F.Cu) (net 6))
 (segment (start 146.794399 70.283231) (end 143.07763 74) (width 0.3048) (layer F.Cu) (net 6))
 (segment (start 144.5 76.5) (end 142 74) (width 0.3048) (layer F.Cu) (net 6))
 (segment (start 146.451 58.6105) (end 146.4535 58.613) (width 0.3048) (layer F.Cu) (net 5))
 (segment (start 144.272 58.6105) (end 146.451 58.6105) (width 0.3048) (layer F.Cu) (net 5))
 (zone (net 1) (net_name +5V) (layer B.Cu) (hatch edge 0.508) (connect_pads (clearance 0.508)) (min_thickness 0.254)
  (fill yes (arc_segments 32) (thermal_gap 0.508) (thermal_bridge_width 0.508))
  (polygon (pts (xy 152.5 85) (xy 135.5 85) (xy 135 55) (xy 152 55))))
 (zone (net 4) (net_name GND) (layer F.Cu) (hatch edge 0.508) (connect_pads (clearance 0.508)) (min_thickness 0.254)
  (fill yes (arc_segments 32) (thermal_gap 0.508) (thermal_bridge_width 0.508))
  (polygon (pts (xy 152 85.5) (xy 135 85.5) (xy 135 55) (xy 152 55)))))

